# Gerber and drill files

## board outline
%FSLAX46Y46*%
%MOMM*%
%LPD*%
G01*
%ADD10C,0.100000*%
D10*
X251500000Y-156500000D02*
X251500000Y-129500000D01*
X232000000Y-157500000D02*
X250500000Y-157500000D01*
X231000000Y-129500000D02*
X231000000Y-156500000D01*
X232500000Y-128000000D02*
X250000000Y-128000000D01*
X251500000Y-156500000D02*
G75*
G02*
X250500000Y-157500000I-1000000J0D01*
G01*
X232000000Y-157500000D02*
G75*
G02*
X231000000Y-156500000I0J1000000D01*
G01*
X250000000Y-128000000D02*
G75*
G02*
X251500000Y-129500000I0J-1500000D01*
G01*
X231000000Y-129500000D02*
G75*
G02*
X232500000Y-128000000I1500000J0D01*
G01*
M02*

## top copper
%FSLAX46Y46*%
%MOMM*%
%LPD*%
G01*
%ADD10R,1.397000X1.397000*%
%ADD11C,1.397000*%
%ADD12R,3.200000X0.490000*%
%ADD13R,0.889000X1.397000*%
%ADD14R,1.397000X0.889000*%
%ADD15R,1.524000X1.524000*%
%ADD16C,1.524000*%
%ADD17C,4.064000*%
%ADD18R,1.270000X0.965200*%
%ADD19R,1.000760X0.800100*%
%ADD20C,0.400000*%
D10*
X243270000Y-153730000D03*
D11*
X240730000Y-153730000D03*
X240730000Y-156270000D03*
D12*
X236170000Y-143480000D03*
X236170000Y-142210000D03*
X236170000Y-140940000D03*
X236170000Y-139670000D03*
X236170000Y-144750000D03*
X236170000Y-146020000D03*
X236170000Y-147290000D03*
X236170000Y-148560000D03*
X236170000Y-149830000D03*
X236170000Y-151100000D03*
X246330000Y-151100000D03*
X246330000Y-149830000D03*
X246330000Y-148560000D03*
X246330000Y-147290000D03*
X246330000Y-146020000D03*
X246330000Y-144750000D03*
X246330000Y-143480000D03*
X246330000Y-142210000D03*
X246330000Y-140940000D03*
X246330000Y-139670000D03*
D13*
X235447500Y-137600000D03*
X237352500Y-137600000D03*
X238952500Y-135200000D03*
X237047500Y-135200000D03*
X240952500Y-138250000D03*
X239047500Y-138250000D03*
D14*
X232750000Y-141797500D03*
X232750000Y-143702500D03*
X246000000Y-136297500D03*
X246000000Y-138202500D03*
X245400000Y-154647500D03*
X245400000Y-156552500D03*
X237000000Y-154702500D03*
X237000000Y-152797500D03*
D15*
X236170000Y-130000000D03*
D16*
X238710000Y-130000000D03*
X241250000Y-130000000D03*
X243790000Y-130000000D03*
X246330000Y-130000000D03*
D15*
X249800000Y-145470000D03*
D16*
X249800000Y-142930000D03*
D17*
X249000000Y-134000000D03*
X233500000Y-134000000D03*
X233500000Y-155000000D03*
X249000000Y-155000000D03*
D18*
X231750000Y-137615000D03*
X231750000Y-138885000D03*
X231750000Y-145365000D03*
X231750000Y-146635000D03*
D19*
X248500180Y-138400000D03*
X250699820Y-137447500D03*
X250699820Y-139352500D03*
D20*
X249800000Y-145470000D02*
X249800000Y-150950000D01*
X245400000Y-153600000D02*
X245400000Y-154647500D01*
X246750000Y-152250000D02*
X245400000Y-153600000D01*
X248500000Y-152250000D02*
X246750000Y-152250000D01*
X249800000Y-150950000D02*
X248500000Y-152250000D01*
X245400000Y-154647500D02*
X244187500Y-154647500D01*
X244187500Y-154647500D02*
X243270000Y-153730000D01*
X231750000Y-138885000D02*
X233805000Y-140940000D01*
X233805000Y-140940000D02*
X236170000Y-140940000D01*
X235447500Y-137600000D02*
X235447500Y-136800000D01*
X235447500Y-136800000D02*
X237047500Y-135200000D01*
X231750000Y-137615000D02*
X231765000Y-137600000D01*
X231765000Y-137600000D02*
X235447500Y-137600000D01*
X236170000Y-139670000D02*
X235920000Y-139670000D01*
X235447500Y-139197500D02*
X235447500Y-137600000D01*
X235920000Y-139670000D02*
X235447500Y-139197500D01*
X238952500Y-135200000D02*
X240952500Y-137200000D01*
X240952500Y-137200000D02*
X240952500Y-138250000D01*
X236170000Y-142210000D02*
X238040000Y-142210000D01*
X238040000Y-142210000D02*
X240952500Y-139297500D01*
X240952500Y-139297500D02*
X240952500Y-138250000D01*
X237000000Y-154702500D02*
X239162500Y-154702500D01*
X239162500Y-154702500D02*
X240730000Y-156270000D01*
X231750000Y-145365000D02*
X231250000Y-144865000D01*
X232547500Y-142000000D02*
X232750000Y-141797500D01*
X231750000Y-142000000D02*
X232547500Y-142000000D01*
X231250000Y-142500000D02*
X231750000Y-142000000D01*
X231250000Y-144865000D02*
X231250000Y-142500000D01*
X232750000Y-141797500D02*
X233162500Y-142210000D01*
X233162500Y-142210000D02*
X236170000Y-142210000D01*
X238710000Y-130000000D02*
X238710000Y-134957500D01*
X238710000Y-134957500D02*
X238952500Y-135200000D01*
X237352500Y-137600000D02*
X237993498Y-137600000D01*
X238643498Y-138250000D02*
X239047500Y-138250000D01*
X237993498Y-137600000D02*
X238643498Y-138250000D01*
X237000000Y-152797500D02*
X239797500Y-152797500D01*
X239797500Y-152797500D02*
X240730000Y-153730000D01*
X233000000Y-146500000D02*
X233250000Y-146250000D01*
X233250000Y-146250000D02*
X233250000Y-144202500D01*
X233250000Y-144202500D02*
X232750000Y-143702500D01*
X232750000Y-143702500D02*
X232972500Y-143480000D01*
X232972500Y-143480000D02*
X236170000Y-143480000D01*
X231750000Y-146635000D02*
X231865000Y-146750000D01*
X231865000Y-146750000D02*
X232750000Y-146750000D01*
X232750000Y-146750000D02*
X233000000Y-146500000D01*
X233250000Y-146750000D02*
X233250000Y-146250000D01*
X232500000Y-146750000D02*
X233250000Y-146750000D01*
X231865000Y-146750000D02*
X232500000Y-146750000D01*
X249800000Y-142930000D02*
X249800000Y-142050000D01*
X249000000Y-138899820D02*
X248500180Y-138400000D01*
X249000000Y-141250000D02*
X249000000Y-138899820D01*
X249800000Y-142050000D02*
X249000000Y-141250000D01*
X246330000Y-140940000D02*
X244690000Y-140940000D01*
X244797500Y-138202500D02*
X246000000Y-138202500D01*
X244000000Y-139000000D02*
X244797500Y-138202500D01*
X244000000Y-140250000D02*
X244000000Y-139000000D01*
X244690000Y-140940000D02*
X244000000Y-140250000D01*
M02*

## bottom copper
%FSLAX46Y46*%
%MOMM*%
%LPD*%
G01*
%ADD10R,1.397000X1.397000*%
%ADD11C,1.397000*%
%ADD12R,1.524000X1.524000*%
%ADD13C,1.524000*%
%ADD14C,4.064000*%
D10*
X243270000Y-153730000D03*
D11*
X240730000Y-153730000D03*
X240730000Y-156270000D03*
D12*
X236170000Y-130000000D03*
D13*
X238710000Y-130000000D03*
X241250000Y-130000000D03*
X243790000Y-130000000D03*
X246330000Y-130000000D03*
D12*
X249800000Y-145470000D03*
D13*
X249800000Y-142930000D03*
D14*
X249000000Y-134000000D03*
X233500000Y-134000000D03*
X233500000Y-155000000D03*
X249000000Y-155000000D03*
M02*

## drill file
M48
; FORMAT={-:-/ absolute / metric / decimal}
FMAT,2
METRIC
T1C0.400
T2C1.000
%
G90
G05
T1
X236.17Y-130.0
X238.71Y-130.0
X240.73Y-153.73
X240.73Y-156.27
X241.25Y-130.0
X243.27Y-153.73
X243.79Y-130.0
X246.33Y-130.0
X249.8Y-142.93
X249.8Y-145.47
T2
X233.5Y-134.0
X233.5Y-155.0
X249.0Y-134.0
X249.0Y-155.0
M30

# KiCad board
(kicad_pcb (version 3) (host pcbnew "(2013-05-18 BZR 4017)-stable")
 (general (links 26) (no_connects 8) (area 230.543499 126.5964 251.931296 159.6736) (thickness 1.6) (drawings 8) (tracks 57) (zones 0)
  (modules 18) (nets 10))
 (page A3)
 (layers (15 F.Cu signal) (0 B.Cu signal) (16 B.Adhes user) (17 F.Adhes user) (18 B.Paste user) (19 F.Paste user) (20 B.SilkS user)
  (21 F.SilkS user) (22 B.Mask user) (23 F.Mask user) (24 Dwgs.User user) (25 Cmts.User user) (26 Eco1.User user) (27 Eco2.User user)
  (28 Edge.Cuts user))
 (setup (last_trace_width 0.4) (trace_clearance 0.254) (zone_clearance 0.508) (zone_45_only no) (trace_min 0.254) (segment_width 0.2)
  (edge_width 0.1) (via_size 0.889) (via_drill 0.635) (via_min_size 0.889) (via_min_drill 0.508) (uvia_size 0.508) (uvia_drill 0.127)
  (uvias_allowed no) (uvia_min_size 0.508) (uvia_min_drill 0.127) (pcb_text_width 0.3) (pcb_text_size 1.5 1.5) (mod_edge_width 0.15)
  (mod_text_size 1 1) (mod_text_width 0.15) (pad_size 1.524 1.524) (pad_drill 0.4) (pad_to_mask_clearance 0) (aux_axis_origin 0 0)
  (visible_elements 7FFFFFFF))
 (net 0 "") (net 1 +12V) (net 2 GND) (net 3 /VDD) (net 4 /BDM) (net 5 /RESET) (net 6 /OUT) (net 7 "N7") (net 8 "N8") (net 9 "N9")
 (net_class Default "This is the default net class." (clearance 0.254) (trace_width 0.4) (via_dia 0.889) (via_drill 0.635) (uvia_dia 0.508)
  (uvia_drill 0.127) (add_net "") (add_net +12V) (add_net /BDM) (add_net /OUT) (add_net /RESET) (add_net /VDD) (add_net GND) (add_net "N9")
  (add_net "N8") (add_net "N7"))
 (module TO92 (layer F.Cu) (at 242 155)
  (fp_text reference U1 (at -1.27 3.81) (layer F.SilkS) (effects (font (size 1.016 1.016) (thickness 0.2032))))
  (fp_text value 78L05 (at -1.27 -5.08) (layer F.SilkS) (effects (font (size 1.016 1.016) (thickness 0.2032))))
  (pad 1 thru_hole rect (at 1.27 -1.27) (size 1.397 1.397) (drill 0.4) (layers *.Cu *.Mask F.SilkS) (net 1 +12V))
  (pad 2 thru_hole circle (at -1.27 -1.27) (size 1.397 1.397) (drill 0.4) (layers *.Cu *.Mask F.SilkS) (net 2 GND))
  (pad 3 thru_hole circle (at -1.27 1.27) (size 1.397 1.397) (drill 0.4) (layers *.Cu *.Mask F.SilkS) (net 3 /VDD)))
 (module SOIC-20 (layer F.Cu) (at 241.25 144.75)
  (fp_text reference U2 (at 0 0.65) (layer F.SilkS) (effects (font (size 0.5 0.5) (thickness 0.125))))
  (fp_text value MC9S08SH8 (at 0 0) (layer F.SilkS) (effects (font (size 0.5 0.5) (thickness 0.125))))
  (pad 4 smd rect (at -5.08 -1.27) (size 3.2 0.49) (layers F.Cu F.Paste F.Mask) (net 2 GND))
  (pad 3 smd rect (at -5.08 -2.54) (size 3.2 0.49) (layers F.Cu F.Paste F.Mask) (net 3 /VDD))
  (pad 2 smd rect (at -5.08 -3.81) (size 3.2 0.49) (layers F.Cu F.Paste F.Mask) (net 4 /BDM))
  (pad 1 smd rect (at -5.08 -5.08) (size 3.2 0.49) (layers F.Cu F.Paste F.Mask) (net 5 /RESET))
  (pad 5 smd rect (at -5.08 0) (size 3.2 0.49) (layers F.Cu F.Paste F.Mask))
  (pad 6 smd rect (at -5.08 1.27) (size 3.2 0.49) (layers F.Cu F.Paste F.Mask))
  (pad 7 smd rect (at -5.08 2.54) (size 3.2 0.49) (layers F.Cu F.Paste F.Mask))
  (pad 8 smd rect (at -5.08 3.81) (size 3.2 0.49) (layers F.Cu F.Paste F.Mask))
  (pad 9 smd rect (at -5.08 5.08) (size 3.2 0.49) (layers F.Cu F.Paste F.Mask))
  (pad 10 smd rect (at -5.08 6.35) (size 3.2 0.49) (layers F.Cu F.Paste F.Mask))
  (pad 11 smd rect (at 5.08 6.35) (size 3.2 0.49) (layers F.Cu F.Paste F.Mask))
  (pad 12 smd rect (at 5.08 5.08) (size 3.2 0.49) (layers F.Cu F.Paste F.Mask) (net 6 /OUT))
  (pad 13 smd rect (at 5.08 3.81) (size 3.2 0.49) (layers F.Cu F.Paste F.Mask))
  (pad 14 smd rect (at 5.08 2.54) (size 3.2 0.49) (layers F.Cu F.Paste F.Mask))
  (pad 15 smd rect (at 5.08 1.27) (size 3.2 0.49) (layers F.Cu F.Paste F.Mask))
  (pad 16 smd rect (at 5.08 0) (size 3.2 0.49) (layers F.Cu F.Paste F.Mask))
  (pad 17 smd rect (at 5.08 -1.27) (size 3.2 0.49) (layers F.Cu F.Paste F.Mask))
  (pad 18 smd rect (at 5.08 -2.54) (size 3.2 0.49) (layers F.Cu F.Paste F.Mask))
  (pad 19 smd rect (at 5.08 -3.81) (size 3.2 0.49) (layers F.Cu F.Paste F.Mask) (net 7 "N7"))
  (pad 20 smd rect (at 5.08 -5.08) (size 3.2 0.49) (layers F.Cu F.Paste F.Mask)))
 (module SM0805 (layer F.Cu) (at 236.4 137.6)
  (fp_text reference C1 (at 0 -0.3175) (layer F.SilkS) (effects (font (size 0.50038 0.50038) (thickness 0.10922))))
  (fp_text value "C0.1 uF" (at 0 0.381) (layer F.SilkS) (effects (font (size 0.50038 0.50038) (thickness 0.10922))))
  (pad 1 smd rect (at -0.9525 0) (size 0.889 1.397) (layers F.Cu F.Paste F.Mask) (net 5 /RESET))
  (pad 2 smd rect (at 0.9525 0) (size 0.889 1.397) (layers F.Cu F.Paste F.Mask) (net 2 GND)))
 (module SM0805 (layer F.Cu) (at 238 135.2 180)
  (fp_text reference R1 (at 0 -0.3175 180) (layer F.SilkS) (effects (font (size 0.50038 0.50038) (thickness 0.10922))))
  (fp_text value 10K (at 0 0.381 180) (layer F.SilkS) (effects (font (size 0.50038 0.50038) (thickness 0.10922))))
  (pad 1 smd rect (at -0.9525 0 180) (size 0.889 1.397) (layers F.Cu F.Paste F.Mask) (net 3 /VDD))
  (pad 2 smd rect (at 0.9525 0 180) (size 0.889 1.397) (layers F.Cu F.Paste F.Mask) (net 5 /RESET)))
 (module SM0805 (layer F.Cu) (at 240 138.25 180)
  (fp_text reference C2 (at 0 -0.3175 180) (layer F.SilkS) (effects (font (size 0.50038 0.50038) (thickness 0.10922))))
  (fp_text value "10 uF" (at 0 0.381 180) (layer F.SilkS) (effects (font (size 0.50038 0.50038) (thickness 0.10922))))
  (pad 1 smd rect (at -0.9525 0 180) (size 0.889 1.397) (layers F.Cu F.Paste F.Mask) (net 3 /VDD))
  (pad 2 smd rect (at 0.9525 0 180) (size 0.889 1.397) (layers F.Cu F.Paste F.Mask) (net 2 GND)))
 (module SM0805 (layer F.Cu) (at 232.75 142.75 270)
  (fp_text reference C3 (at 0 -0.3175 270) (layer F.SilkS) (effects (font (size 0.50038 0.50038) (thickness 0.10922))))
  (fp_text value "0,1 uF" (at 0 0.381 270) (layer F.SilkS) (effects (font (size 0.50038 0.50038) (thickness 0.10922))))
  (pad 1 smd rect (at -0.9525 0 270) (size 0.889 1.397) (layers F.Cu F.Paste F.Mask) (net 3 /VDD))
  (pad 2 smd rect (at 0.9525 0 270) (size 0.889 1.397) (layers F.Cu F.Paste F.Mask) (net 2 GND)))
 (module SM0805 (layer F.Cu) (at 246 137.25 270)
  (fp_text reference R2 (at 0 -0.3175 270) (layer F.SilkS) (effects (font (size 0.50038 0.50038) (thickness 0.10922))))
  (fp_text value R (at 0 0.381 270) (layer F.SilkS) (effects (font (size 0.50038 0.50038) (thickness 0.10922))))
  (pad 1 smd rect (at -0.9525 0 270) (size 0.889 1.397) (layers F.Cu F.Paste F.Mask) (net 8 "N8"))
  (pad 2 smd rect (at 0.9525 0 270) (size 0.889 1.397) (layers F.Cu F.Paste F.Mask) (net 7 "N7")))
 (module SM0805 (layer F.Cu) (at 245.4 155.6 270)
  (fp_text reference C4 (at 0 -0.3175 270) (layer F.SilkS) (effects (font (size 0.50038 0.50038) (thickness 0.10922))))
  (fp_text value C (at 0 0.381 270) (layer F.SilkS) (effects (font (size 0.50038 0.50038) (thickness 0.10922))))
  (pad 1 smd rect (at -0.9525 0 270) (size 0.889 1.397) (layers F.Cu F.Paste F.Mask) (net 1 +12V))
  (pad 2 smd rect (at 0.9525 0 270) (size 0.889 1.397) (layers F.Cu F.Paste F.Mask) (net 2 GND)))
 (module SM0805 (layer F.Cu) (at 237 153.75 90)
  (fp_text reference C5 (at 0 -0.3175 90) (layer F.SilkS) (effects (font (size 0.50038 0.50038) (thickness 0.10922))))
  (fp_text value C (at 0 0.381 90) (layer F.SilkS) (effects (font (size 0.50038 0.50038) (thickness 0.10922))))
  (pad 1 smd rect (at -0.9525 0 90) (size 0.889 1.397) (layers F.Cu F.Paste F.Mask) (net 3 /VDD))
  (pad 2 smd rect (at 0.9525 0 90) (size 0.889 1.397) (layers F.Cu F.Paste F.Mask) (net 2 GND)))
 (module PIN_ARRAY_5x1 (layer F.Cu) (at 241.25 130)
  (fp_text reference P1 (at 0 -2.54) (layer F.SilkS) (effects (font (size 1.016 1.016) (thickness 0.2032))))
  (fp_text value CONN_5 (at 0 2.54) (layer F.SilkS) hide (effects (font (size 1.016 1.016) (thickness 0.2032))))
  (pad 1 thru_hole rect (at -5.08 0) (size 1.524 1.524) (drill 0.4) (layers *.Cu *.Mask F.SilkS))
  (pad 2 thru_hole circle (at -2.54 0) (size 1.524 1.524) (drill 0.4) (layers *.Cu *.Mask F.SilkS) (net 3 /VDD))
  (pad 3 thru_hole circle (at 0 0) (size 1.524 1.524) (drill 0.4) (layers *.Cu *.Mask F.SilkS))
  (pad 4 thru_hole circle (at 2.54 0) (size 1.524 1.524) (drill 0.4) (layers *.Cu *.Mask F.SilkS) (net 6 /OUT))
  (pad 5 thru_hole circle (at 5.08 0) (size 1.524 1.524) (drill 0.4) (layers *.Cu *.Mask F.SilkS) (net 2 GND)))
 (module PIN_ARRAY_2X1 (layer F.Cu) (at 249.8 144.2 90)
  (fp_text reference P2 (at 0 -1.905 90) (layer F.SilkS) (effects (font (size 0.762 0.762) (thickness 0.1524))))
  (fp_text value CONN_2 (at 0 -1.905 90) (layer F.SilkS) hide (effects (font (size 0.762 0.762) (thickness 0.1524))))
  (pad 1 thru_hole rect (at -1.27 0 90) (size 1.524 1.524) (drill 0.4) (layers *.Cu *.Mask F.SilkS) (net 1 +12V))
  (pad 2 thru_hole circle (at 1.27 0 90) (size 1.524 1.524) (drill 0.4) (layers *.Cu *.Mask F.SilkS) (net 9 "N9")))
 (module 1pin (layer F.Cu) (at 249 134)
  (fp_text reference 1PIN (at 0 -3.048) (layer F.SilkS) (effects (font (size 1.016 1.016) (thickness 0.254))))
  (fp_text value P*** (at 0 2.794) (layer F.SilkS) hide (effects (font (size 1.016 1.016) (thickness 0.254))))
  (pad 1 thru_hole circle (at 0 0) (size 4.064 4.064) (drill 1) (layers *.Cu *.Mask F.SilkS)))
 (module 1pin (layer F.Cu) (at 233.5 134)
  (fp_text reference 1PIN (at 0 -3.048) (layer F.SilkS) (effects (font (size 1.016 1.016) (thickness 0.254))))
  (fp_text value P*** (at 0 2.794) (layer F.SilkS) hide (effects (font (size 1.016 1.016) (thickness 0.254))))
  (pad 1 thru_hole circle (at 0 0) (size 4.064 4.064) (drill 1) (layers *.Cu *.Mask F.SilkS)))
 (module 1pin (layer F.Cu) (at 233.5 155)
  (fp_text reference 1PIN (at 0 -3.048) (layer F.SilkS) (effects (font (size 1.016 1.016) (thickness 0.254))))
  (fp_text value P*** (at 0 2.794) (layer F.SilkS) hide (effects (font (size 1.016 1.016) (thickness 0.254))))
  (pad 1 thru_hole circle (at 0 0) (size 4.064 4.064) (drill 1) (layers *.Cu *.Mask F.SilkS)))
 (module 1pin (layer F.Cu) (at 249 155)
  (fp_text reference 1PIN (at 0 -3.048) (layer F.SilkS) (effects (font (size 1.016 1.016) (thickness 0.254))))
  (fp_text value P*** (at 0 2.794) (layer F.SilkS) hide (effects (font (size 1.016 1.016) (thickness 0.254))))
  (pad 1 thru_hole circle (at 0 0) (size 4.064 4.064) (drill 1) (layers *.Cu *.Mask F.SilkS)))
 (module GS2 (layer F.Cu) (at 231.75 138.25)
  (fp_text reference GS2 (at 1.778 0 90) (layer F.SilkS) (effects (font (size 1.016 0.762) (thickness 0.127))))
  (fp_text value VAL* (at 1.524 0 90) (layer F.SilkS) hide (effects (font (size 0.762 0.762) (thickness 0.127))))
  (pad 1 smd rect (at 0 -0.635) (size 1.27 0.9652) (layers F.Cu F.Paste F.Mask) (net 5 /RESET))
  (pad 2 smd rect (at 0 0.635) (size 1.27 0.9652) (layers F.Cu F.Paste F.Mask) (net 4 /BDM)))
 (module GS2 (layer F.Cu) (at 231.75 146)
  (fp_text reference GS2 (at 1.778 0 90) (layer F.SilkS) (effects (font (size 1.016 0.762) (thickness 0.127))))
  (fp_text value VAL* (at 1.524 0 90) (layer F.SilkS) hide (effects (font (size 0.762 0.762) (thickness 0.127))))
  (pad 1 smd rect (at 0 -0.635) (size 1.27 0.9652) (layers F.Cu F.Paste F.Mask) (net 3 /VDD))
  (pad 2 smd rect (at 0 0.635) (size 1.27 0.9652) (layers F.Cu F.Paste F.Mask) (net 2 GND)))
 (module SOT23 (layer F.Cu) (at 249.6 138.4 90)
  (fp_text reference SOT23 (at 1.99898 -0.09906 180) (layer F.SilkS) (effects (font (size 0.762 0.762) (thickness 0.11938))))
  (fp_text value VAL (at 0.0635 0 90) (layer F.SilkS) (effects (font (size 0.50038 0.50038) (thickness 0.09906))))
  (pad 3 smd rect (at 0 -1.09982 90) (size 0.8001 1.00076) (layers F.Cu F.Paste F.Mask) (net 9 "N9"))
  (pad 2 smd rect (at 0.9525 1.09982 90) (size 0.8001 1.00076) (layers F.Cu F.Paste F.Mask) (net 2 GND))
  (pad 1 smd rect (at -0.9525 1.09982 90) (size 0.8001 1.00076) (layers F.Cu F.Paste F.Mask) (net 8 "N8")))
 (gr_line (start 251.5 156.5) (end 251.5 129.5) (angle 90) (layer Edge.Cuts) (width 0.1))
 (gr_line (start 232 157.5) (end 250.5 157.5) (angle 90) (layer Edge.Cuts) (width 0.1))
 (gr_line (start 231 129.5) (end 231 156.5) (angle 90) (layer Edge.Cuts) (width 0.1))
 (gr_line (start 232.5 128) (end 250 128) (angle 90) (layer Edge.Cuts) (width 0.1))
 (gr_arc (start 250.5 156.5) (end 251.5 156.5) (angle 90) (layer Edge.Cuts) (width 0.1))
 (gr_arc (start 232 156.5) (end 232 157.5) (angle 90) (layer Edge.Cuts) (width 0.1))
 (gr_arc (start 250 129.5) (end 250 128) (angle 90) (layer Edge.Cuts) (width 0.1))
 (gr_arc (start 232.5 129.5) (end 231 129.5) (angle 90) (layer Edge.Cuts) (width 0.1))
 (segment (start 249.8 145.47) (end 249.8 150.95) (width 0.4) (layer F.Cu) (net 1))
 (segment (start 245.4 153.6) (end 245.4 154.6475) (width 0.4) (layer F.Cu) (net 1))
 (segment (start 246.75 152.25) (end 245.4 153.6) (width 0.4) (layer F.Cu) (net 1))
 (segment (start 248.5 152.25) (end 246.75 152.25) (width 0.4) (layer F.Cu) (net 1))
 (segment (start 249.8 150.95) (end 248.5 152.25) (width 0.4) (layer F.Cu) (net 1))
 (segment (start 245.4 154.6475) (end 244.1875 154.6475) (width 0.4) (layer F.Cu) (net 1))
 (segment (start 244.1875 154.6475) (end 243.27 153.73) (width 0.4) (layer F.Cu) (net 1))
 (segment (start 231.75 138.885) (end 233.805 140.94) (width 0.4) (layer F.Cu) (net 4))
 (segment (start 233.805 140.94) (end 236.17 140.94) (width 0.4) (layer F.Cu) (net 4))
 (segment (start 235.4475 137.6) (end 235.4475 136.8) (width 0.4) (layer F.Cu) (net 5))
 (segment (start 235.4475 136.8) (end 237.0475 135.2) (width 0.4) (layer F.Cu) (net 5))
 (segment (start 231.75 137.615) (end 231.765 137.6) (width 0.4) (layer F.Cu) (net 5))
 (segment (start 231.765 137.6) (end 235.4475 137.6) (width 0.4) (layer F.Cu) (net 5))
 (segment (start 236.17 139.67) (end 235.92 139.67) (width 0.4) (layer F.Cu) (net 5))
 (segment (start 235.4475 139.1975) (end 235.4475 137.6) (width 0.4) (layer F.Cu) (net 5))
 (segment (start 235.92 139.67) (end 235.4475 139.1975) (width 0.4) (layer F.Cu) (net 5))
 (segment (start 238.9525 135.2) (end 240.9525 137.2) (width 0.4) (layer F.Cu) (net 3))
 (segment (start 240.9525 137.2) (end 240.9525 138.25) (width 0.4) (layer F.Cu) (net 3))
 (segment (start 236.17 142.21) (end 238.04 142.21) (width 0.4) (layer F.Cu) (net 3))
 (segment (start 238.04 142.21) (end 240.9525 139.2975) (width 0.4) (layer F.Cu) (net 3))
 (segment (start 240.9525 139.2975) (end 240.9525 138.25) (width 0.4) (layer F.Cu) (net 3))
 (segment (start 237 154.7025) (end 239.1625 154.7025) (width 0.4) (layer F.Cu) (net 3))
 (segment (start 239.1625 154.7025) (end 240.73 156.27) (width 0.4) (layer F.Cu) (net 3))
 (segment (start 231.75 145.365) (end 231.25 144.865) (width 0.4) (layer F.Cu) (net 3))
 (segment (start 232.5475 142) (end 232.75 141.7975) (width 0.4) (layer F.Cu) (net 3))
 (segment (start 231.75 142) (end 232.5475 142) (width 0.4) (layer F.Cu) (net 3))
 (segment (start 231.25 142.5) (end 231.75 142) (width 0.4) (layer F.Cu) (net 3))
 (segment (start 231.25 144.865) (end 231.25 142.5) (width 0.4) (layer F.Cu) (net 3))
 (segment (start 232.75 141.7975) (end 233.1625 142.21) (width 0.4) (layer F.Cu) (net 3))
 (segment (start 233.1625 142.21) (end 236.17 142.21) (width 0.4) (layer F.Cu) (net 3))
 (segment (start 238.71 130) (end 238.71 134.9575) (width 0.4) (layer F.Cu) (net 3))
 (segment (start 238.71 134.9575) (end 238.9525 135.2) (width 0.4) (layer F.Cu) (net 3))
 (segment (start 237.3525 137.6) (end 237.993498 137.6) (width 0.4) (layer F.Cu) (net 2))
 (segment (start 238.643498 138.25) (end 239.0475 138.25) (width 0.4) (layer F.Cu) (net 2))
 (segment (start 237.993498 137.6) (end 238.643498 138.25) (width 0.4) (layer F.Cu) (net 2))
 (segment (start 237 152.7975) (end 239.7975 152.7975) (width 0.4) (layer F.Cu) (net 2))
 (segment (start 239.7975 152.7975) (end 240.73 153.73) (width 0.4) (layer F.Cu) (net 2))
 (segment (start 233 146.5) (end 233.25 146.25) (width 0.4) (layer F.Cu) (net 2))
 (segment (start 233.25 146.25) (end 233.25 144.2025) (width 0.4) (layer F.Cu) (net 2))
 (segment (start 233.25 144.2025) (end 232.75 143.7025) (width 0.4) (layer F.Cu) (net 2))
 (segment (start 232.75 143.7025) (end 232.9725 143.48) (width 0.4) (layer F.Cu) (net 2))
 (segment (start 232.9725 143.48) (end 236.17 143.48) (width 0.4) (layer F.Cu) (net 2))
 (segment (start 231.75 146.635) (end 231.865 146.75) (width 0.4) (layer F.Cu) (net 2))
 (segment (start 231.865 146.75) (end 232.75 146.75) (width 0.4) (layer F.Cu) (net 2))
 (segment (start 232.75 146.75) (end 233 146.5) (width 0.4) (layer F.Cu) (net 2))
 (segment (start 233.25 146.75) (end 233.25 146.25) (width 0.4) (layer F.Cu) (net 2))
 (segment (start 232.5 146.75) (end 233.25 146.75) (width 0.4) (layer F.Cu) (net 2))
 (segment (start 231.865 146.75) (end 232.5 146.75) (width 0.4) (layer F.Cu) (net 2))
 (segment (start 249.8 142.93) (end 249.8 142.05) (width 0.4) (layer F.Cu) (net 9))
 (segment (start 249 138.89982) (end 248.50018 138.4) (width 0.4) (layer F.Cu) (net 9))
 (segment (start 249 141.25) (end 249 138.89982) (width 0.4) (layer F.Cu) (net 9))
 (segment (start 249.8 142.05) (end 249 141.25) (width 0.4) (layer F.Cu) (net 9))
 (segment (start 246.33 140.94) (end 244.69 140.94) (width 0.4) (layer F.Cu) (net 7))
 (segment (start 244.7975 138.2025) (end 246 138.2025) (width 0.4) (layer F.Cu) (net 7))
 (segment (start 244 139) (end 244.7975 138.2025) (width 0.4) (layer F.Cu) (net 7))
 (segment (start 244 140.25) (end 244 139) (width 0.4) (layer F.Cu) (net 7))
 (segment (start 244.69 140.94) (end 244 140.25) (width 0.4) (layer F.Cu) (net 7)))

